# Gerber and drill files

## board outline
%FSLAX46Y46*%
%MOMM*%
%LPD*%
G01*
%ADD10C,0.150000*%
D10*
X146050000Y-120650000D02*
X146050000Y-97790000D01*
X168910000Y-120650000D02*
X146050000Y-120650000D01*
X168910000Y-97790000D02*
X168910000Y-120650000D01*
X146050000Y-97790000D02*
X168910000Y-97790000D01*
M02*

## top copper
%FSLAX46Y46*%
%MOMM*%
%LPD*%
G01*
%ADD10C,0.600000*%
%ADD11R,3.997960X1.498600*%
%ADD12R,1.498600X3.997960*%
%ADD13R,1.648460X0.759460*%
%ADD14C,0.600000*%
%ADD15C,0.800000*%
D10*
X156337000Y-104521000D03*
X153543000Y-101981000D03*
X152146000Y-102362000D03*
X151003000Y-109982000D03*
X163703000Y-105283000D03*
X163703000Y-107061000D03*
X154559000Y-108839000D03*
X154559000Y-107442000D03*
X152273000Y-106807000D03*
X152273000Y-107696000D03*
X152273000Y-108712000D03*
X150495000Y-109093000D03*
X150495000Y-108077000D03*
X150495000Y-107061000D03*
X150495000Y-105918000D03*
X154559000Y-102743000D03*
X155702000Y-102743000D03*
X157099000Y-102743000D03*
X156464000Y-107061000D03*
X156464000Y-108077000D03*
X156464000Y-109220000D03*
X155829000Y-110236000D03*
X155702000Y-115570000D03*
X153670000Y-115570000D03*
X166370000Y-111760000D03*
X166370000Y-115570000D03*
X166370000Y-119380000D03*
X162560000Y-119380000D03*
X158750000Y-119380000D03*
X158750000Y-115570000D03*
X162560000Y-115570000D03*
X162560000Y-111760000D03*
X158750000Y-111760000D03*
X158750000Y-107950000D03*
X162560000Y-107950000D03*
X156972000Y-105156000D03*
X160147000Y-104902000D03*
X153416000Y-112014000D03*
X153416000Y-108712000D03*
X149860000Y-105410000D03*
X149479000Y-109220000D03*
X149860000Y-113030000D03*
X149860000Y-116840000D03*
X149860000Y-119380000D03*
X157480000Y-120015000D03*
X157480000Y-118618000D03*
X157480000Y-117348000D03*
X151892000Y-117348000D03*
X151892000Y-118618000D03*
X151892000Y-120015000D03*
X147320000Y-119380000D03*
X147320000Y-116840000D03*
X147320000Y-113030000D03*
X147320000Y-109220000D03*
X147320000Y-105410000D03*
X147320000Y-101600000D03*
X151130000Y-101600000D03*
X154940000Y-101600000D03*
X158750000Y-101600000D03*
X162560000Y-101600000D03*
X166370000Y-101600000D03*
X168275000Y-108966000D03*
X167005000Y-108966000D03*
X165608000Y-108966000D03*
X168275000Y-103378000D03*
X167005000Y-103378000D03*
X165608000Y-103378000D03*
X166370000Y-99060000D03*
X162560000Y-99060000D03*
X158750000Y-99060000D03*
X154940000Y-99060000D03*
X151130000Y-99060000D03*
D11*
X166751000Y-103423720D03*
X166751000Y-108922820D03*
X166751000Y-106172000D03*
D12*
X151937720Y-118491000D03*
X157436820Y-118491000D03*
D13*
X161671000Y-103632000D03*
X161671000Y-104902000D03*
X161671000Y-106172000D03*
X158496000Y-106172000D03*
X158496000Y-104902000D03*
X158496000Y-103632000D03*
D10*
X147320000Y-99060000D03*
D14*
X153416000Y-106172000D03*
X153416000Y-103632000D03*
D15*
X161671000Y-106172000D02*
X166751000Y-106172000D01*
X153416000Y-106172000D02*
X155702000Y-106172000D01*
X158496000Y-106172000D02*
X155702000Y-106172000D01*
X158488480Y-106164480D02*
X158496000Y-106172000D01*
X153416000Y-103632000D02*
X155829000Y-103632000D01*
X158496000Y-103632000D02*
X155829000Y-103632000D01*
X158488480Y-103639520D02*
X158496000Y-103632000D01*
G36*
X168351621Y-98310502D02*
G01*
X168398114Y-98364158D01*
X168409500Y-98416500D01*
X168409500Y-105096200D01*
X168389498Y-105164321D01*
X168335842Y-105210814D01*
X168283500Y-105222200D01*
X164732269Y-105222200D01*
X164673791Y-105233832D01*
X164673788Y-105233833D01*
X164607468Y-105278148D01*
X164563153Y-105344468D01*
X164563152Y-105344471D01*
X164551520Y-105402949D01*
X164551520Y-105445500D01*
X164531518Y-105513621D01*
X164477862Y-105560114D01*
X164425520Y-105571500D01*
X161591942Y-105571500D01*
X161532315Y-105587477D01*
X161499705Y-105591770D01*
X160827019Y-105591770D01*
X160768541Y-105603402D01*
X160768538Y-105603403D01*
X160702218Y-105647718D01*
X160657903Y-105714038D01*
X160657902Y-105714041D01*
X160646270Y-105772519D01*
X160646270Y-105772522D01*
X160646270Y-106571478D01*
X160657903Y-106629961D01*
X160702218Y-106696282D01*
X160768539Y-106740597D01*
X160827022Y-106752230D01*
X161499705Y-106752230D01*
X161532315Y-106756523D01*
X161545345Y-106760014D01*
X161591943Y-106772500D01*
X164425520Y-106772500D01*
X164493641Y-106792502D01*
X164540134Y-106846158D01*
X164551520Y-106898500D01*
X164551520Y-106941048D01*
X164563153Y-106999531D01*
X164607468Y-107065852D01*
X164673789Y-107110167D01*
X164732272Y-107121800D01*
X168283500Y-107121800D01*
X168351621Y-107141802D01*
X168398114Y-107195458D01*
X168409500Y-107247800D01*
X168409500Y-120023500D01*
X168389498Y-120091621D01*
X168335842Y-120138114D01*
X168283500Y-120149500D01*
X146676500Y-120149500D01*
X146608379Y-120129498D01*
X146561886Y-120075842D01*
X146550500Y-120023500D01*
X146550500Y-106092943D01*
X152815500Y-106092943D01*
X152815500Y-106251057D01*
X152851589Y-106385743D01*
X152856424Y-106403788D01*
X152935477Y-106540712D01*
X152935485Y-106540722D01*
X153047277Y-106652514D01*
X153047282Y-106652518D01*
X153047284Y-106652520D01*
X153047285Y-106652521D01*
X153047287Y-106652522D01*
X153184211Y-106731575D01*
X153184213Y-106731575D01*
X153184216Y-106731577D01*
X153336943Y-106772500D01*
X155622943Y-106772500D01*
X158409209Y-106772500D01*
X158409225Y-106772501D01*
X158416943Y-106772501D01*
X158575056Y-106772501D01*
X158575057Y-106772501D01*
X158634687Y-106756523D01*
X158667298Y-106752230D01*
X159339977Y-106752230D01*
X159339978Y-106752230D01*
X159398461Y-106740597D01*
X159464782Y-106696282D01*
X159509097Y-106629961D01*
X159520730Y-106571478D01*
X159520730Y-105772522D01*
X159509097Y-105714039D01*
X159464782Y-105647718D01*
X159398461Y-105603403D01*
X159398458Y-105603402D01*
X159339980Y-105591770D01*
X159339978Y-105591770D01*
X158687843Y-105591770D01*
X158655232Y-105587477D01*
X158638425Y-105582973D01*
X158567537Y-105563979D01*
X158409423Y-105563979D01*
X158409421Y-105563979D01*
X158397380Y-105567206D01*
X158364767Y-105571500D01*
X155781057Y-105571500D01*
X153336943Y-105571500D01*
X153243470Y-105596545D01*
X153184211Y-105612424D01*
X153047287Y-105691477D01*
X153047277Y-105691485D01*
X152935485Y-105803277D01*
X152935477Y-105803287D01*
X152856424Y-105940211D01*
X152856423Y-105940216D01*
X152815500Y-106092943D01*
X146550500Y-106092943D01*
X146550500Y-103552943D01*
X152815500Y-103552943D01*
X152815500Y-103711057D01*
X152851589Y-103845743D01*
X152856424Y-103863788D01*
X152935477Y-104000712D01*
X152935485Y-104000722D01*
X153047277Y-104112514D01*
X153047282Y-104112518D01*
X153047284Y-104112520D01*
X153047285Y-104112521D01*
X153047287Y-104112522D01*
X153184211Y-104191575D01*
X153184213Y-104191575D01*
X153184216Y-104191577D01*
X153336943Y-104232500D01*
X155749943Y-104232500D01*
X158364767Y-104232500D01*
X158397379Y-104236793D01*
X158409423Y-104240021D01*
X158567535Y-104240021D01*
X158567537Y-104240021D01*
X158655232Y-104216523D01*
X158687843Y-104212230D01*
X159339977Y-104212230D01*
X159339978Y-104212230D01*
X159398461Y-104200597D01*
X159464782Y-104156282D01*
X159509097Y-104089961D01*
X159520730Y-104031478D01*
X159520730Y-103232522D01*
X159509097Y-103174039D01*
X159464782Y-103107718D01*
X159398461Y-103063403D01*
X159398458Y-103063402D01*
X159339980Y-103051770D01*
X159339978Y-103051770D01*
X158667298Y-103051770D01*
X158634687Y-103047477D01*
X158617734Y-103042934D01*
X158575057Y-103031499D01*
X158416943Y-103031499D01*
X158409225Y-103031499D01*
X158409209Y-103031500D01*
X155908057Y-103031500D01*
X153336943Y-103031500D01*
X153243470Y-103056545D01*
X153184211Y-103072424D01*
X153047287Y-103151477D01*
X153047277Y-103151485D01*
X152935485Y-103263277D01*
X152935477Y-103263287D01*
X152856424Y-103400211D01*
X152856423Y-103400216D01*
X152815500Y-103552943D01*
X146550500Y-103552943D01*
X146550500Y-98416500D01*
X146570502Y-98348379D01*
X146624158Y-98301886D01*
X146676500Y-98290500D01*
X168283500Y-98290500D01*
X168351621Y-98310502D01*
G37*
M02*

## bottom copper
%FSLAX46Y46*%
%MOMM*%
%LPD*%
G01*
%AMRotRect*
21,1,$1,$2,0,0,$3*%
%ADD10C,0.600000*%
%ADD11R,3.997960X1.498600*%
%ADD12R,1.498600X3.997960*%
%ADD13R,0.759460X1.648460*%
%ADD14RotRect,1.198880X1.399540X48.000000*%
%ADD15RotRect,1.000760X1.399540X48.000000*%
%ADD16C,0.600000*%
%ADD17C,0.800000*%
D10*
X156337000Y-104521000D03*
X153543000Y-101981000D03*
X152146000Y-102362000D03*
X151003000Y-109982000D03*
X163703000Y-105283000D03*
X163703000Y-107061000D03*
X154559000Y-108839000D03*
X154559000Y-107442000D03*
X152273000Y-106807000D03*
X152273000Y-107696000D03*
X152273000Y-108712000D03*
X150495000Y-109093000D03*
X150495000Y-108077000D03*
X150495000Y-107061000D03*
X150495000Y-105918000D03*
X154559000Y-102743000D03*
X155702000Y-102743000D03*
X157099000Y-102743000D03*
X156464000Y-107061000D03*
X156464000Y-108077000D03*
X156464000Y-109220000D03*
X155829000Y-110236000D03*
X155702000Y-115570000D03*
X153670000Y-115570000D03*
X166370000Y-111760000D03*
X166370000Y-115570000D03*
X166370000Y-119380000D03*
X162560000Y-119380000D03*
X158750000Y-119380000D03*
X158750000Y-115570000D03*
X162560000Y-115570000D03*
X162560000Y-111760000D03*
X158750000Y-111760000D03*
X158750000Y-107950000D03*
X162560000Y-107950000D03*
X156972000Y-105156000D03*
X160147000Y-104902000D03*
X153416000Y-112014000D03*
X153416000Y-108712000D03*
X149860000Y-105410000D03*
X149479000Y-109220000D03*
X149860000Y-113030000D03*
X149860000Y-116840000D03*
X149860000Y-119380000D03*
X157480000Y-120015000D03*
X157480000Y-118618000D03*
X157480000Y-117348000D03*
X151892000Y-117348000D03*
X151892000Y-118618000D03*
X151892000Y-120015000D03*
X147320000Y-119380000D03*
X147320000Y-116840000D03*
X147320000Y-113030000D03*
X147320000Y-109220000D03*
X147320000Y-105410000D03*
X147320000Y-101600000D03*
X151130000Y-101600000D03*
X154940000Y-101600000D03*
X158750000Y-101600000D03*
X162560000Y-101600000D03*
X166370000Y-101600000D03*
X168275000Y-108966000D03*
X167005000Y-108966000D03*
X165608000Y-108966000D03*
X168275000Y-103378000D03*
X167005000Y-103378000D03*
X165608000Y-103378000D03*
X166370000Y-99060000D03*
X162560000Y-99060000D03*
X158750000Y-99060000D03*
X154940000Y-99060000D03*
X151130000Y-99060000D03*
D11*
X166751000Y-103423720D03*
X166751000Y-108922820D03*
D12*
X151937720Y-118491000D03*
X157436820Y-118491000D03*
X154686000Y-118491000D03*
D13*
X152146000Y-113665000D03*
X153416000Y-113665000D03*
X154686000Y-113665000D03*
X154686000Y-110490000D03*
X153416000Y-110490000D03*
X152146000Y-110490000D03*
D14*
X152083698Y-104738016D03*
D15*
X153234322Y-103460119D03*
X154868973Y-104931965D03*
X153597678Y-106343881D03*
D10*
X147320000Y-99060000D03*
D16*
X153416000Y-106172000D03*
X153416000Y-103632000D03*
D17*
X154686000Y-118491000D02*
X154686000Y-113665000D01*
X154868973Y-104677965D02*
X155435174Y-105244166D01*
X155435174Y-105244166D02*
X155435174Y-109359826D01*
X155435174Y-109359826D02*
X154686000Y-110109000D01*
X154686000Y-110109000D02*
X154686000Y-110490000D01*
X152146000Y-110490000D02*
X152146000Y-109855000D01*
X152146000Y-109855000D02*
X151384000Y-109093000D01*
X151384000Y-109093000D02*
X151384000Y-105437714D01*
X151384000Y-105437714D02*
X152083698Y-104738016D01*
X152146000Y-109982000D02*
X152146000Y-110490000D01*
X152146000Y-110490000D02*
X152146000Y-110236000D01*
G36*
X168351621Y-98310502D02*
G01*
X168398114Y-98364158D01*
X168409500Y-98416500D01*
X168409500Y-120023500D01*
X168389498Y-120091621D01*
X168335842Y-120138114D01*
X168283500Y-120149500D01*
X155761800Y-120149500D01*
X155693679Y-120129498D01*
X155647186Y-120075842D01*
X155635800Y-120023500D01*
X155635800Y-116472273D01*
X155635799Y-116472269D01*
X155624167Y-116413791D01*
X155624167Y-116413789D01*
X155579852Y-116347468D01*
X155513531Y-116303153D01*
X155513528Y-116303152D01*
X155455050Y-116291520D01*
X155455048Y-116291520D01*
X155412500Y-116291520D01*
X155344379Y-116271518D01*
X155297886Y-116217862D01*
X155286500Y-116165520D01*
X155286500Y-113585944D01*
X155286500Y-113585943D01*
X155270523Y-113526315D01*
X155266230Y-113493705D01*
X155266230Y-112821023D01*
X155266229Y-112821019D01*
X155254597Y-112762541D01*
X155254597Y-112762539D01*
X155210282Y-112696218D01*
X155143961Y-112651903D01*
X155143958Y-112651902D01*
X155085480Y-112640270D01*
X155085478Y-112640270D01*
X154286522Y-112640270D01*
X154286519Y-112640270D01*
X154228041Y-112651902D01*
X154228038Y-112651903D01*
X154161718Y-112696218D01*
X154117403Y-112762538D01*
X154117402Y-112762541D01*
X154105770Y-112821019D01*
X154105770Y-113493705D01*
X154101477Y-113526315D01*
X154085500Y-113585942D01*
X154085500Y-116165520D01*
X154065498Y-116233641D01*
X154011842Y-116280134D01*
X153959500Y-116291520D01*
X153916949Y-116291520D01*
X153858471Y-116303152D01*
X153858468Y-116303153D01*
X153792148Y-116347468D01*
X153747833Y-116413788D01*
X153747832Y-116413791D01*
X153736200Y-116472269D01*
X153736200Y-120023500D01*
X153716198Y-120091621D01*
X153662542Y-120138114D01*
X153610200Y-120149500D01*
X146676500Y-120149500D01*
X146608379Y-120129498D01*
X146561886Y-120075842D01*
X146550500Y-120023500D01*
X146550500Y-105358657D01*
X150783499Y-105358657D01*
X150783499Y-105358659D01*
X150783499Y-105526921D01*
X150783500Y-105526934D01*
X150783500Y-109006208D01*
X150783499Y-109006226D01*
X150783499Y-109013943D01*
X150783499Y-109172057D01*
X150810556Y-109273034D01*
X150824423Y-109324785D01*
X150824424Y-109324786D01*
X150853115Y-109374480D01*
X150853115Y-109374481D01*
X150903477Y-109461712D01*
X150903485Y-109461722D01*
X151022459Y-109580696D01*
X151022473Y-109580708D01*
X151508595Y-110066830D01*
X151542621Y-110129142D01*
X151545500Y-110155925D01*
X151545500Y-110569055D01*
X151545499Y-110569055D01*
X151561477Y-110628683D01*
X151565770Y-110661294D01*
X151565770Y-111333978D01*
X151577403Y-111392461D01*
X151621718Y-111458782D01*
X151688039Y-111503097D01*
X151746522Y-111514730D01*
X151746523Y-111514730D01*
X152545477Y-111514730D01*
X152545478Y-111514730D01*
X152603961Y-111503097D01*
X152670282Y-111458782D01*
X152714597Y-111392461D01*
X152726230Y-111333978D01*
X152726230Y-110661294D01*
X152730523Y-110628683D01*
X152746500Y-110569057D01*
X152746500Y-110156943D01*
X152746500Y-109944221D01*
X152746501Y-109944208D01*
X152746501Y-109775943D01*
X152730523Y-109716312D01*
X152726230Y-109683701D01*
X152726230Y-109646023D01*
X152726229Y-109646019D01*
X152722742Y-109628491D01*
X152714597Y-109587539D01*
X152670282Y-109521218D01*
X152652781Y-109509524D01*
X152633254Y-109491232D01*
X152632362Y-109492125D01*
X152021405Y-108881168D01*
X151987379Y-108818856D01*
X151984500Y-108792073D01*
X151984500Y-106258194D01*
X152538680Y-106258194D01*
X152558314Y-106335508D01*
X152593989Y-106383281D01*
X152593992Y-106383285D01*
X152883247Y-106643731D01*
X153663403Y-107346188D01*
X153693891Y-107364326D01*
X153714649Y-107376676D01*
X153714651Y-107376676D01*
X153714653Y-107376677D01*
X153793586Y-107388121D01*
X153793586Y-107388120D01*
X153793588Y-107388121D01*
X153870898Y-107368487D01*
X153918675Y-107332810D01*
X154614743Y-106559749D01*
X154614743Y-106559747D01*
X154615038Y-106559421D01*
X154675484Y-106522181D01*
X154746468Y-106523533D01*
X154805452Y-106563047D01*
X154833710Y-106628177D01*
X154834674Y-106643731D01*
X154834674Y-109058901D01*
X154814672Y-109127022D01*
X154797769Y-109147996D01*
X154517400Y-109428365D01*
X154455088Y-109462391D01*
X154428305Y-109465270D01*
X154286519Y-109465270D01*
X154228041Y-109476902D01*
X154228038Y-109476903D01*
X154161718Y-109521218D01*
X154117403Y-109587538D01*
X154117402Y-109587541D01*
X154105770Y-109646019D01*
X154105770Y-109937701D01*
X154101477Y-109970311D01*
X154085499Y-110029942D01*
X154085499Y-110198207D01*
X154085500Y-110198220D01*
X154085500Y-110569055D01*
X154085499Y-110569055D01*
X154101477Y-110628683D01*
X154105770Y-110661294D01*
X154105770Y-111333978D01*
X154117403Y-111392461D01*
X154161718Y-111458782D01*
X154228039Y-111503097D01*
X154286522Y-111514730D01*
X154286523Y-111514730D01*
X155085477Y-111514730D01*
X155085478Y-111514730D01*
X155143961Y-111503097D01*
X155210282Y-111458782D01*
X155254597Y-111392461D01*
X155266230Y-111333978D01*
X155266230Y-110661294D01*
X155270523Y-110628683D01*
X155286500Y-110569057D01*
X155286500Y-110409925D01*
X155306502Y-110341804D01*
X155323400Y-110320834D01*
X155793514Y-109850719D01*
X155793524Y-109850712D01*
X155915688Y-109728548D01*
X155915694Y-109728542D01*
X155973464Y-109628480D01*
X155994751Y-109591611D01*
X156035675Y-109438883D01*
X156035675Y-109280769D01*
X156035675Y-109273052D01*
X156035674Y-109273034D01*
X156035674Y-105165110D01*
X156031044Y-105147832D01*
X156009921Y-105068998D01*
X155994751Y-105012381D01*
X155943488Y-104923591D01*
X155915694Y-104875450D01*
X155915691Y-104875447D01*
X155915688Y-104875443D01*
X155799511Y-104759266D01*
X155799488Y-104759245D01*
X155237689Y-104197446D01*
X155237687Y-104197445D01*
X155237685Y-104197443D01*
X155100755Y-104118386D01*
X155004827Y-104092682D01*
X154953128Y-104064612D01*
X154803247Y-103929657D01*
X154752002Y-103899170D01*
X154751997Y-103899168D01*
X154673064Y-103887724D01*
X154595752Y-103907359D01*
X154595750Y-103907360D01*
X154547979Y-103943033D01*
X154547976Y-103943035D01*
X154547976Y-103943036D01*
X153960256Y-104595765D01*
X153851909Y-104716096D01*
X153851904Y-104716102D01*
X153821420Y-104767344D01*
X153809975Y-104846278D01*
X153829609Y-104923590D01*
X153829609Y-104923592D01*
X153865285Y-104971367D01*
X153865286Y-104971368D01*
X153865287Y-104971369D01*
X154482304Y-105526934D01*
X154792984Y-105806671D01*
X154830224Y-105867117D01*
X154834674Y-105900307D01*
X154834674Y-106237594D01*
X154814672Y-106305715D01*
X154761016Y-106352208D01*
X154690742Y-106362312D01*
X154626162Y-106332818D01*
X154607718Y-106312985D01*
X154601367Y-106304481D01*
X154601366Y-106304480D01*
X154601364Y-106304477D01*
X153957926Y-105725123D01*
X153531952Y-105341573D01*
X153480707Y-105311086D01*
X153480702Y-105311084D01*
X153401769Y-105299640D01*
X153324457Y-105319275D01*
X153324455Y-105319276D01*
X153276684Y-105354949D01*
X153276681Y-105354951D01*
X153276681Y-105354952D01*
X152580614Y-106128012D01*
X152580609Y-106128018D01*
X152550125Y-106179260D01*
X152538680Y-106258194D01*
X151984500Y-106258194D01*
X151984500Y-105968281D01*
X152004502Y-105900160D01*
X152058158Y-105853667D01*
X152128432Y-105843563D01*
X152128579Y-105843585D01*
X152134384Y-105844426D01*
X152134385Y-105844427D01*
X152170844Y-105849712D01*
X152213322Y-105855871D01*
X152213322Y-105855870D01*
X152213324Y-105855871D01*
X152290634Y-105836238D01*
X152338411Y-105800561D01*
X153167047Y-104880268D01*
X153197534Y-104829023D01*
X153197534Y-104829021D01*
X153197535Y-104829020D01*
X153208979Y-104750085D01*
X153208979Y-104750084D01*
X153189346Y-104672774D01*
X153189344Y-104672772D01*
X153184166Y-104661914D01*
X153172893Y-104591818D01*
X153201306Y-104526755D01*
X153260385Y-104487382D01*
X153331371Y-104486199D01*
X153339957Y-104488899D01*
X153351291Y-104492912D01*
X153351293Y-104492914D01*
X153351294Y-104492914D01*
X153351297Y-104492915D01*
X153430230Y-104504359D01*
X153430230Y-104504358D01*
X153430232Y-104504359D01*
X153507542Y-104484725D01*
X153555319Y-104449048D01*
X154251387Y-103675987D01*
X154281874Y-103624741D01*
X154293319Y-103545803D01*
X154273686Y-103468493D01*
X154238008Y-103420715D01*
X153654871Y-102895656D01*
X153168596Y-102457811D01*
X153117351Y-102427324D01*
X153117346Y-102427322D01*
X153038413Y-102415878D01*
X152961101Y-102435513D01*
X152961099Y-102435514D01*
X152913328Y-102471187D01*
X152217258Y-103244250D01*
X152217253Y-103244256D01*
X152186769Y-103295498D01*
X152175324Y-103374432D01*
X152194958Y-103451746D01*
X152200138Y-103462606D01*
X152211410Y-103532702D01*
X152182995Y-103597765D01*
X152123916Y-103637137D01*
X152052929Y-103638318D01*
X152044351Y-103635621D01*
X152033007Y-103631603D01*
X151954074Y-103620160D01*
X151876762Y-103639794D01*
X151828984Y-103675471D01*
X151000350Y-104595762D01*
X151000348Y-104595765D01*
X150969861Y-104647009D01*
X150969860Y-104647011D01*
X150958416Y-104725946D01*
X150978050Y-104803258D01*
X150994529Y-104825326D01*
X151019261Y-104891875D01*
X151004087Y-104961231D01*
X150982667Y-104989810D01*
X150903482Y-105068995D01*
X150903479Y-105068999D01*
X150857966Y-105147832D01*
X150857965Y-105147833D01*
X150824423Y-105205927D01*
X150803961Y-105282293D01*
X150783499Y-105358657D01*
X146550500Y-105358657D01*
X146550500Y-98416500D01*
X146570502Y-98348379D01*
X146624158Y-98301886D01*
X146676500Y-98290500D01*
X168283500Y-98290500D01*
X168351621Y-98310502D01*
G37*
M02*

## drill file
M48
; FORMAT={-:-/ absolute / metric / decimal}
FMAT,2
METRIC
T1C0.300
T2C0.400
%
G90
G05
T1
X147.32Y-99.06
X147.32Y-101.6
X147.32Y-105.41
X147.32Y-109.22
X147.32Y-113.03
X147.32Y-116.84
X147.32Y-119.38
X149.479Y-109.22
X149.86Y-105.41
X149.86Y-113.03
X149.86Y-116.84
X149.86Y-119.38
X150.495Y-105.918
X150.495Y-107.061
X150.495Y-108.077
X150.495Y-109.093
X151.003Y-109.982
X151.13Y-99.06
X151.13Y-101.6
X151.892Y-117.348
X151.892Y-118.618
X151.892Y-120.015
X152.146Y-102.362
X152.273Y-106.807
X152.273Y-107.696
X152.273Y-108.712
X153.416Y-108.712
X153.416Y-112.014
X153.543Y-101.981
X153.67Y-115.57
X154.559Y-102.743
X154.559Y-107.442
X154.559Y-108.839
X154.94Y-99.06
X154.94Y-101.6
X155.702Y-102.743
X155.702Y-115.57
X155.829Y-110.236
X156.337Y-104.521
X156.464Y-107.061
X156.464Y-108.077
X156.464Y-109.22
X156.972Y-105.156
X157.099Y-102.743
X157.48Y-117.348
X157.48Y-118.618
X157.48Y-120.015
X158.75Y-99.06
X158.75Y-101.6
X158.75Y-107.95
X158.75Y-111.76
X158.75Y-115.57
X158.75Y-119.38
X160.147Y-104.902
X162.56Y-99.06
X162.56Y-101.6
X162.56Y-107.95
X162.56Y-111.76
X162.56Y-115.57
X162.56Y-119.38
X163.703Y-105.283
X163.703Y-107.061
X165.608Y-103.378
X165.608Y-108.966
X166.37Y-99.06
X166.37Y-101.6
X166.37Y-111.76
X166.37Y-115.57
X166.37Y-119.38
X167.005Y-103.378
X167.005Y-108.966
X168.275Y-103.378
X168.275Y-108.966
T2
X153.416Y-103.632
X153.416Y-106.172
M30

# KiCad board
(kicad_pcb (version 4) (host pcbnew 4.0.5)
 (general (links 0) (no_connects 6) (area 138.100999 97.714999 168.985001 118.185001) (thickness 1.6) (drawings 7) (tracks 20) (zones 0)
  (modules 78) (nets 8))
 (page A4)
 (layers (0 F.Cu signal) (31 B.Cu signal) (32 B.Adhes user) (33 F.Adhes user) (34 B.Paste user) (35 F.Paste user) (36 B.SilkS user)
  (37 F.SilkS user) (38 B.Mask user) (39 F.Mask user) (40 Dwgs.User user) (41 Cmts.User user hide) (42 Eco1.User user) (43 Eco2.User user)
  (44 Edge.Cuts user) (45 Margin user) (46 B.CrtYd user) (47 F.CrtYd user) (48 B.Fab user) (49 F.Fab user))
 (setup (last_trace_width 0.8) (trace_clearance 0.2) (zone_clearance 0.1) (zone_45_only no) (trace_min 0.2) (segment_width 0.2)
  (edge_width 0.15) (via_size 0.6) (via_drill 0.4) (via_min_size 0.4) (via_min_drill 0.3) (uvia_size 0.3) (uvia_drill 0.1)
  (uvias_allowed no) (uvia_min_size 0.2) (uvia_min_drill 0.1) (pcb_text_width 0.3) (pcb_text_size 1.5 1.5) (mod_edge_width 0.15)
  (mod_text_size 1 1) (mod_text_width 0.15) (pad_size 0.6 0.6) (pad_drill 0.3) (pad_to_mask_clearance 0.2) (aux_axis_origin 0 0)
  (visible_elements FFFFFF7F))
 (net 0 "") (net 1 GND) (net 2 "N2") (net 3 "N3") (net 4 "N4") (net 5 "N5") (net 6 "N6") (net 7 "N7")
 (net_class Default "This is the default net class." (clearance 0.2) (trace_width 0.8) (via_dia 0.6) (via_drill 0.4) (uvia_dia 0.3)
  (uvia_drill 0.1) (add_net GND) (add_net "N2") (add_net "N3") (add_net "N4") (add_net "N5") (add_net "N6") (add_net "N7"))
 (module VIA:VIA (layer F.Cu) (at 156.337 104.521)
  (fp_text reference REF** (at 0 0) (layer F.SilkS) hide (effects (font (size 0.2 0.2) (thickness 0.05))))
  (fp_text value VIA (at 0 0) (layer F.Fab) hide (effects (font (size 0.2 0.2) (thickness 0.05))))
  (pad 1 thru_hole circle (at 0 0) (size 0.6 0.6) (drill 0.3) (layers *.Cu) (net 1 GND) (zone_connect 2)))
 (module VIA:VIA (layer F.Cu) (at 153.543 101.981)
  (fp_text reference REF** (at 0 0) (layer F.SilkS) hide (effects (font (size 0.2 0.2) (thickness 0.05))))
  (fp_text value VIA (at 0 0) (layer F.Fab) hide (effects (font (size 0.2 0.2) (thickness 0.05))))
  (pad 1 thru_hole circle (at 0 0) (size 0.6 0.6) (drill 0.3) (layers *.Cu) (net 1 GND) (zone_connect 2)))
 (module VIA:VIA (layer F.Cu) (at 152.146 102.362)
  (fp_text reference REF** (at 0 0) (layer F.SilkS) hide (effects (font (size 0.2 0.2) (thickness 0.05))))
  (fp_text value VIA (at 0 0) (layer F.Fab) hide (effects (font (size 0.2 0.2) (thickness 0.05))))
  (pad 1 thru_hole circle (at 0 0) (size 0.6 0.6) (drill 0.3) (layers *.Cu) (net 1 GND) (zone_connect 2)))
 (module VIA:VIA (layer F.Cu) (at 151.003 109.982)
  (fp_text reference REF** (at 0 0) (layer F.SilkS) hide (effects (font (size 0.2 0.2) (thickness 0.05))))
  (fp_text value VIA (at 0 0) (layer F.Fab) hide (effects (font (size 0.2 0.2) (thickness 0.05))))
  (pad 1 thru_hole circle (at 0 0) (size 0.6 0.6) (drill 0.3) (layers *.Cu) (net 1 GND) (zone_connect 2)))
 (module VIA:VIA (layer F.Cu) (at 163.703 105.283)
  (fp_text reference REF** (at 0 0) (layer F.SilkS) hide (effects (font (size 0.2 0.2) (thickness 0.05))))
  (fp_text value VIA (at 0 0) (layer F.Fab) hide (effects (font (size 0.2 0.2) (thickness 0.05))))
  (pad 1 thru_hole circle (at 0 0) (size 0.6 0.6) (drill 0.3) (layers *.Cu) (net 1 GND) (zone_connect 2)))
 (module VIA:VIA (layer F.Cu) (at 163.703 107.061)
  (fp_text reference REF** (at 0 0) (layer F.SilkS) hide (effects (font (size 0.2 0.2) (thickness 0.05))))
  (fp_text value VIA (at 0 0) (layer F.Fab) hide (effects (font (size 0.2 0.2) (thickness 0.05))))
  (pad 1 thru_hole circle (at 0 0) (size 0.6 0.6) (drill 0.3) (layers *.Cu) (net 1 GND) (zone_connect 2)))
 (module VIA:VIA (layer F.Cu) (at 154.559 108.839)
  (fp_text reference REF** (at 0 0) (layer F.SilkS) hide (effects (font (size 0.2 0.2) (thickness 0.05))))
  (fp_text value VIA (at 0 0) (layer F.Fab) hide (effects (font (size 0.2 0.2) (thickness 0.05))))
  (pad 1 thru_hole circle (at 0 0) (size 0.6 0.6) (drill 0.3) (layers *.Cu) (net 1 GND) (zone_connect 2)))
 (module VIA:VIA (layer F.Cu) (at 154.559 107.442)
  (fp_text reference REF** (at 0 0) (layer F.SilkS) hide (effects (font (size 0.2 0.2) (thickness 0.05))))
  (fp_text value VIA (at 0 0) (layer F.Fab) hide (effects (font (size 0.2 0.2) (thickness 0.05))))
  (pad 1 thru_hole circle (at 0 0) (size 0.6 0.6) (drill 0.3) (layers *.Cu) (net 1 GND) (zone_connect 2)))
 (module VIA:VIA (layer F.Cu) (at 152.273 106.807)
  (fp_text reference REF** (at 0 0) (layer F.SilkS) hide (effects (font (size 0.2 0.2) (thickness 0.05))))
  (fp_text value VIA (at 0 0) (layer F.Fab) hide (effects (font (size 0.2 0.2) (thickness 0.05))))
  (pad 1 thru_hole circle (at 0 0) (size 0.6 0.6) (drill 0.3) (layers *.Cu) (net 1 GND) (zone_connect 2)))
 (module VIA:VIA (layer F.Cu) (at 152.273 107.696)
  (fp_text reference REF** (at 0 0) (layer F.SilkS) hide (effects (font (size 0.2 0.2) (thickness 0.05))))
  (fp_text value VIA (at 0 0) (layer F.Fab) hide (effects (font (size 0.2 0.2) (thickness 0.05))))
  (pad 1 thru_hole circle (at 0 0) (size 0.6 0.6) (drill 0.3) (layers *.Cu) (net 1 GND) (zone_connect 2)))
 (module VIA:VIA (layer F.Cu) (at 152.273 108.712)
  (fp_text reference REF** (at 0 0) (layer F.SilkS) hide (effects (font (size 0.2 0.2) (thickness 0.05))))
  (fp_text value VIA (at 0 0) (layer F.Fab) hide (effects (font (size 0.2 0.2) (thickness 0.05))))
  (pad 1 thru_hole circle (at 0 0) (size 0.6 0.6) (drill 0.3) (layers *.Cu) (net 1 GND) (zone_connect 2)))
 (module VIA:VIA (layer F.Cu) (at 150.495 109.093)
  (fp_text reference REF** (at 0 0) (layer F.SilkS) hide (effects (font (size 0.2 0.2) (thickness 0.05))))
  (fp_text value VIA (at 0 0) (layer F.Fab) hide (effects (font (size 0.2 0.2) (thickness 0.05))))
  (pad 1 thru_hole circle (at 0 0) (size 0.6 0.6) (drill 0.3) (layers *.Cu) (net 1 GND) (zone_connect 2)))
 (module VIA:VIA (layer F.Cu) (at 150.495 108.077)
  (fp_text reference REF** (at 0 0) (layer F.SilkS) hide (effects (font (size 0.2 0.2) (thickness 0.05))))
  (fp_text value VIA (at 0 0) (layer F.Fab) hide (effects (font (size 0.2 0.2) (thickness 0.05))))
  (pad 1 thru_hole circle (at 0 0) (size 0.6 0.6) (drill 0.3) (layers *.Cu) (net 1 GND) (zone_connect 2)))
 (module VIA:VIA (layer F.Cu) (at 150.495 107.061)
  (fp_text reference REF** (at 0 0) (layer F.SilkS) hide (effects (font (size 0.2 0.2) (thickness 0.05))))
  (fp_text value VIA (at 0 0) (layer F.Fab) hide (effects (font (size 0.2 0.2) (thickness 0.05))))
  (pad 1 thru_hole circle (at 0 0) (size 0.6 0.6) (drill 0.3) (layers *.Cu) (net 1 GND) (zone_connect 2)))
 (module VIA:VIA (layer F.Cu) (at 150.495 105.918)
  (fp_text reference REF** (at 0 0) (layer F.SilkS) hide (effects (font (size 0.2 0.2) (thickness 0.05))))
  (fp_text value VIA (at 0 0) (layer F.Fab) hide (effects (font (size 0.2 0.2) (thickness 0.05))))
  (pad 1 thru_hole circle (at 0 0) (size 0.6 0.6) (drill 0.3) (layers *.Cu) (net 1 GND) (zone_connect 2)))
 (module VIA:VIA (layer F.Cu) (at 154.559 102.743)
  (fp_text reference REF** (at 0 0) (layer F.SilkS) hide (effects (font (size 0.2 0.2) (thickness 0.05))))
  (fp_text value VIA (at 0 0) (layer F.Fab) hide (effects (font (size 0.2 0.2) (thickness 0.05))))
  (pad 1 thru_hole circle (at 0 0) (size 0.6 0.6) (drill 0.3) (layers *.Cu) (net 1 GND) (zone_connect 2)))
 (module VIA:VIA (layer F.Cu) (at 155.702 102.743)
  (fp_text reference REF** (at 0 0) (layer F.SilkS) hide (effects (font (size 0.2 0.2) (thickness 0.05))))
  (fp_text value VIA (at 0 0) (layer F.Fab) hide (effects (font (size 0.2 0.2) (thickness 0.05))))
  (pad 1 thru_hole circle (at 0 0) (size 0.6 0.6) (drill 0.3) (layers *.Cu) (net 1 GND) (zone_connect 2)))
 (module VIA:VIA (layer F.Cu) (at 157.099 102.743)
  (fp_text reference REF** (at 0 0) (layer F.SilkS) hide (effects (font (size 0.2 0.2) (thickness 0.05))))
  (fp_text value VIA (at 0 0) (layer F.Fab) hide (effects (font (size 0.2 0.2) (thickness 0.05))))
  (pad 1 thru_hole circle (at 0 0) (size 0.6 0.6) (drill 0.3) (layers *.Cu) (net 1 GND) (zone_connect 2)))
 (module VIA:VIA (layer F.Cu) (at 156.464 107.061)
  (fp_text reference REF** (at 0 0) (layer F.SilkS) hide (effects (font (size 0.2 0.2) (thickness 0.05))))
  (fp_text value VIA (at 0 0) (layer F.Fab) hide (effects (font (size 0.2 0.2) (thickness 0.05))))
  (pad 1 thru_hole circle (at 0 0) (size 0.6 0.6) (drill 0.3) (layers *.Cu) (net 1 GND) (zone_connect 2)))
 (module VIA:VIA (layer F.Cu) (at 156.464 108.077)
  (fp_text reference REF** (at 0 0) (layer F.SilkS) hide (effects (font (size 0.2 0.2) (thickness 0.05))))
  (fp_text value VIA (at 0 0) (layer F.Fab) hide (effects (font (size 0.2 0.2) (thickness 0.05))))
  (pad 1 thru_hole circle (at 0 0) (size 0.6 0.6) (drill 0.3) (layers *.Cu) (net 1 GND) (zone_connect 2)))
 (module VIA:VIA (layer F.Cu) (at 156.464 109.22)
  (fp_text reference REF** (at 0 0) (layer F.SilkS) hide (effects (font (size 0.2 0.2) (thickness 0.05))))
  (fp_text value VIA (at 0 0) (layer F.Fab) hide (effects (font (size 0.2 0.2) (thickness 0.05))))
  (pad 1 thru_hole circle (at 0 0) (size 0.6 0.6) (drill 0.3) (layers *.Cu) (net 1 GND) (zone_connect 2)))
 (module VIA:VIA (layer F.Cu) (at 155.829 110.236)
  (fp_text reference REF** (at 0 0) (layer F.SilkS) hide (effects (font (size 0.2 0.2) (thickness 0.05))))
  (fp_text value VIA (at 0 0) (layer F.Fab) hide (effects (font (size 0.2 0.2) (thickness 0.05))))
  (pad 1 thru_hole circle (at 0 0) (size 0.6 0.6) (drill 0.3) (layers *.Cu) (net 1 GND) (zone_connect 2)))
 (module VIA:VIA (layer F.Cu) (at 155.702 115.57)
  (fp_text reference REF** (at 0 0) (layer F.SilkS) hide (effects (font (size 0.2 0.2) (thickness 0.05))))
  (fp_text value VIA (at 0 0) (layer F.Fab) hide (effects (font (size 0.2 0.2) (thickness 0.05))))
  (pad 1 thru_hole circle (at 0 0) (size 0.6 0.6) (drill 0.3) (layers *.Cu) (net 1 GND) (zone_connect 2)))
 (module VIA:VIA (layer F.Cu) (at 153.67 115.57)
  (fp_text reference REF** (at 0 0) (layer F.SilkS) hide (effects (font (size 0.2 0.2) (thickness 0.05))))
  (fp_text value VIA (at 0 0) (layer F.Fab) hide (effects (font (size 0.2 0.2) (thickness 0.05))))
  (pad 1 thru_hole circle (at 0 0) (size 0.6 0.6) (drill 0.3) (layers *.Cu) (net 1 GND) (zone_connect 2)))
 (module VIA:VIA (layer F.Cu) (at 166.37 111.76)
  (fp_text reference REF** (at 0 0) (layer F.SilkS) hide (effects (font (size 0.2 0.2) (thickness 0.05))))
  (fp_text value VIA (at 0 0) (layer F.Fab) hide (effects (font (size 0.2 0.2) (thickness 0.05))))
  (pad 1 thru_hole circle (at 0 0) (size 0.6 0.6) (drill 0.3) (layers *.Cu) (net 1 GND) (zone_connect 2)))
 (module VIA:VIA (layer F.Cu) (at 166.37 115.57)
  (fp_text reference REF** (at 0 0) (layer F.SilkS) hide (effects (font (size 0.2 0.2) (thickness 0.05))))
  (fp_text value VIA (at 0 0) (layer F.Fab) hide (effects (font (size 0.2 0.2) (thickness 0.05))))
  (pad 1 thru_hole circle (at 0 0) (size 0.6 0.6) (drill 0.3) (layers *.Cu) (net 1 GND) (zone_connect 2)))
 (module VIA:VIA (layer F.Cu) (at 166.37 119.38)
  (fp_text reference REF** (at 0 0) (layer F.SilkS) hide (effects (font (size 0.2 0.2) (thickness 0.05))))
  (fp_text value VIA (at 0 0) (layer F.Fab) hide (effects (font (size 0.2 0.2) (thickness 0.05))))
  (pad 1 thru_hole circle (at 0 0) (size 0.6 0.6) (drill 0.3) (layers *.Cu) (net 1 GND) (zone_connect 2)))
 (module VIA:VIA (layer F.Cu) (at 162.56 119.38)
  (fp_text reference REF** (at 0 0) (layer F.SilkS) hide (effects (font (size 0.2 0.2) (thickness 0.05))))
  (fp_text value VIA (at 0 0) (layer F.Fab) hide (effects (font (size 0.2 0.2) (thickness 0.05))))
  (pad 1 thru_hole circle (at 0 0) (size 0.6 0.6) (drill 0.3) (layers *.Cu) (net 1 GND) (zone_connect 2)))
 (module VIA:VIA (layer F.Cu) (at 158.75 119.38)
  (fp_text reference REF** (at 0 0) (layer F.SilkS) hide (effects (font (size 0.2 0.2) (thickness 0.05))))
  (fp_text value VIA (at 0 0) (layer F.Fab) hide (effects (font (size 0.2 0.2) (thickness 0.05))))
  (pad 1 thru_hole circle (at 0 0) (size 0.6 0.6) (drill 0.3) (layers *.Cu) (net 1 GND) (zone_connect 2)))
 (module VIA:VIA (layer F.Cu) (at 158.75 115.57)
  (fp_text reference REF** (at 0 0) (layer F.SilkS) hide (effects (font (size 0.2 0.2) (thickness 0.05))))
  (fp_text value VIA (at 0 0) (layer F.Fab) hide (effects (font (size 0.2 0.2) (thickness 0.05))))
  (pad 1 thru_hole circle (at 0 0) (size 0.6 0.6) (drill 0.3) (layers *.Cu) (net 1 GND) (zone_connect 2)))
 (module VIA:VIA (layer F.Cu) (at 162.56 115.57)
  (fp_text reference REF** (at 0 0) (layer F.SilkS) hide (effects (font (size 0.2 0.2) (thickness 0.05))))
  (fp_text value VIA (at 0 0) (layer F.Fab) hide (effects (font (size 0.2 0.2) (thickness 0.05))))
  (pad 1 thru_hole circle (at 0 0) (size 0.6 0.6) (drill 0.3) (layers *.Cu) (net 1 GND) (zone_connect 2)))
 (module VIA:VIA (layer F.Cu) (at 162.56 111.76)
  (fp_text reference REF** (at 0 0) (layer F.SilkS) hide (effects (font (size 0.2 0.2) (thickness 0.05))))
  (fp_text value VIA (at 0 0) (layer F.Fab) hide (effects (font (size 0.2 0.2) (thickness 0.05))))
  (pad 1 thru_hole circle (at 0 0) (size 0.6 0.6) (drill 0.3) (layers *.Cu) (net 1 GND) (zone_connect 2)))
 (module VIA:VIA (layer F.Cu) (at 158.75 111.76)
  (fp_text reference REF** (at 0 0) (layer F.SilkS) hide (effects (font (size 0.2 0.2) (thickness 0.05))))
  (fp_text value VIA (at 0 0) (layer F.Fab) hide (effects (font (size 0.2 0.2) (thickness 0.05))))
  (pad 1 thru_hole circle (at 0 0) (size 0.6 0.6) (drill 0.3) (layers *.Cu) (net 1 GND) (zone_connect 2)))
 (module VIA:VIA (layer F.Cu) (at 158.75 107.95)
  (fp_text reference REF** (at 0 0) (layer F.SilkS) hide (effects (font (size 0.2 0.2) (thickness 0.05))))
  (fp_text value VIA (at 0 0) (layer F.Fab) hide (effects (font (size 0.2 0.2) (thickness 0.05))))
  (pad 1 thru_hole circle (at 0 0) (size 0.6 0.6) (drill 0.3) (layers *.Cu) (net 1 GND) (zone_connect 2)))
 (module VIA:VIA (layer F.Cu) (at 162.56 107.95)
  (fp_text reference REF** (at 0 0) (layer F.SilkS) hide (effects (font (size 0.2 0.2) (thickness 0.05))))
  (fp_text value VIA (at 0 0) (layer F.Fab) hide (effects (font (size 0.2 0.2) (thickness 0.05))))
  (pad 1 thru_hole circle (at 0 0) (size 0.6 0.6) (drill 0.3) (layers *.Cu) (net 1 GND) (zone_connect 2)))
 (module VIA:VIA (layer F.Cu) (at 156.972 105.156)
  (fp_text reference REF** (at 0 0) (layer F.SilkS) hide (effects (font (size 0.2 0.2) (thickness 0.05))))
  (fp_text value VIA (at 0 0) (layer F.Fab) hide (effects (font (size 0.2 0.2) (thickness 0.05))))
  (pad 1 thru_hole circle (at 0 0) (size 0.6 0.6) (drill 0.3) (layers *.Cu) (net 1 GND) (zone_connect 2)))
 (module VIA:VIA (layer F.Cu) (at 160.147 104.902)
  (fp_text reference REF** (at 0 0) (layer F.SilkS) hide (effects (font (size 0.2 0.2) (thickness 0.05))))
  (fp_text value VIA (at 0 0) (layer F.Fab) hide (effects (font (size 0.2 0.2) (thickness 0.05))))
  (pad 1 thru_hole circle (at 0 0) (size 0.6 0.6) (drill 0.3) (layers *.Cu) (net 1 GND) (zone_connect 2)))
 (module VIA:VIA (layer F.Cu) (at 153.416 112.014)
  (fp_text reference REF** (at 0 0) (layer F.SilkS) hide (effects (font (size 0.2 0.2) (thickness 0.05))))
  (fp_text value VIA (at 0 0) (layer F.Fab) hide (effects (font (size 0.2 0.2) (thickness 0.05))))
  (pad 1 thru_hole circle (at 0 0) (size 0.6 0.6) (drill 0.3) (layers *.Cu) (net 1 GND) (zone_connect 2)))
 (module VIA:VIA (layer F.Cu) (at 153.416 108.712)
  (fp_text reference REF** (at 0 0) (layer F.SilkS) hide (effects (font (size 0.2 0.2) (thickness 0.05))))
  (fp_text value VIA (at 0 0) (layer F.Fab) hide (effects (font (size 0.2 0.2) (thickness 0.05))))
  (pad 1 thru_hole circle (at 0 0) (size 0.6 0.6) (drill 0.3) (layers *.Cu) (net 1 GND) (zone_connect 2)))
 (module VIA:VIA (layer F.Cu) (at 149.86 105.41)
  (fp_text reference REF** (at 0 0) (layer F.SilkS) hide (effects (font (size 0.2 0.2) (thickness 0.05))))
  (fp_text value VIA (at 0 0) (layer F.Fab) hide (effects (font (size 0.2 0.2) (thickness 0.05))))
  (pad 1 thru_hole circle (at 0 0) (size 0.6 0.6) (drill 0.3) (layers *.Cu) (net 1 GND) (zone_connect 2)))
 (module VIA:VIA (layer F.Cu) (at 149.479 109.22)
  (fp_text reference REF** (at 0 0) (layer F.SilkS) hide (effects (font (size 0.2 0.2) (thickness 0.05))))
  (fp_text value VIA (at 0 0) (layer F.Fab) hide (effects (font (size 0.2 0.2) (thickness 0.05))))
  (pad 1 thru_hole circle (at 0 0) (size 0.6 0.6) (drill 0.3) (layers *.Cu) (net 1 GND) (zone_connect 2)))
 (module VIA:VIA (layer F.Cu) (at 149.86 113.03)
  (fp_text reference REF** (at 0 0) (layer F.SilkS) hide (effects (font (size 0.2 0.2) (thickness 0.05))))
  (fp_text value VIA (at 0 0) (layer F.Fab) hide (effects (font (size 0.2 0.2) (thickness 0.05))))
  (pad 1 thru_hole circle (at 0 0) (size 0.6 0.6) (drill 0.3) (layers *.Cu) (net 1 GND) (zone_connect 2)))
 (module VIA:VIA (layer F.Cu) (at 149.86 116.84)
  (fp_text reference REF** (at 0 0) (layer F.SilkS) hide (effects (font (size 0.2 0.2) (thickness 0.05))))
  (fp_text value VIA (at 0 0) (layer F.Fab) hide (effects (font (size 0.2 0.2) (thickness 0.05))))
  (pad 1 thru_hole circle (at 0 0) (size 0.6 0.6) (drill 0.3) (layers *.Cu) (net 1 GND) (zone_connect 2)))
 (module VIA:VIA (layer F.Cu) (at 149.86 119.38)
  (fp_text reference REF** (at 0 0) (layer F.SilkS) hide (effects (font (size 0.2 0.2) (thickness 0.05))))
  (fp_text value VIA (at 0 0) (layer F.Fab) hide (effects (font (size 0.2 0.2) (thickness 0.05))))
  (pad 1 thru_hole circle (at 0 0) (size 0.6 0.6) (drill 0.3) (layers *.Cu) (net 1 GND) (zone_connect 2)))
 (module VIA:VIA (layer F.Cu) (at 157.48 120.015)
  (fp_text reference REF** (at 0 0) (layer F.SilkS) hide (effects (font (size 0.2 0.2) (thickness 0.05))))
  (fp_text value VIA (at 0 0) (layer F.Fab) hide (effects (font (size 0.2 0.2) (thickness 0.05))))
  (pad 1 thru_hole circle (at 0 0) (size 0.6 0.6) (drill 0.3) (layers *.Cu) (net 1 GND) (zone_connect 2)))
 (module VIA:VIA (layer F.Cu) (at 157.48 118.618)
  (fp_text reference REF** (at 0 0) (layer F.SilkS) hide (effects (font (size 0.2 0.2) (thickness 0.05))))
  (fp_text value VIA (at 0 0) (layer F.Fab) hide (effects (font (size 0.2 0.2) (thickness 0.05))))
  (pad 1 thru_hole circle (at 0 0) (size 0.6 0.6) (drill 0.3) (layers *.Cu) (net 1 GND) (zone_connect 2)))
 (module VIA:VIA (layer F.Cu) (at 157.48 117.348)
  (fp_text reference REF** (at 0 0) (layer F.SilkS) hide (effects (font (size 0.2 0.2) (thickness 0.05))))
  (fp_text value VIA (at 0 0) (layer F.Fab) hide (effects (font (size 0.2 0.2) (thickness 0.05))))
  (pad 1 thru_hole circle (at 0 0) (size 0.6 0.6) (drill 0.3) (layers *.Cu) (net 1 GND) (zone_connect 2)))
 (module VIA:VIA (layer F.Cu) (at 151.892 117.348)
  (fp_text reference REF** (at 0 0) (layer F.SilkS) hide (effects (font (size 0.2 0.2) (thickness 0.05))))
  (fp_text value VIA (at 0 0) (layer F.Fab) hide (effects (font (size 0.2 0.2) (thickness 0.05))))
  (pad 1 thru_hole circle (at 0 0) (size 0.6 0.6) (drill 0.3) (layers *.Cu) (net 1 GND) (zone_connect 2)))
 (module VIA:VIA (layer F.Cu) (at 151.892 118.618)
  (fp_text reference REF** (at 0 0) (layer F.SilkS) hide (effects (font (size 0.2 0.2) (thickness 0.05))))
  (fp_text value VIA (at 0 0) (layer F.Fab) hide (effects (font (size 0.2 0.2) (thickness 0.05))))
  (pad 1 thru_hole circle (at 0 0) (size 0.6 0.6) (drill 0.3) (layers *.Cu) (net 1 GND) (zone_connect 2)))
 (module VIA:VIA (layer F.Cu) (at 151.892 120.015)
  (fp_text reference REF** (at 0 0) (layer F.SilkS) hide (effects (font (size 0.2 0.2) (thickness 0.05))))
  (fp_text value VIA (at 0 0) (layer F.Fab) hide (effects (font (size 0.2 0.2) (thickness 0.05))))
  (pad 1 thru_hole circle (at 0 0) (size 0.6 0.6) (drill 0.3) (layers *.Cu) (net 1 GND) (zone_connect 2)))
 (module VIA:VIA (layer F.Cu) (at 147.32 119.38)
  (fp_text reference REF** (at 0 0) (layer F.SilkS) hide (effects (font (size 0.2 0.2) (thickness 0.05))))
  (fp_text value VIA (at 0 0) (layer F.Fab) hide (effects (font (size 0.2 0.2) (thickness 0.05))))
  (pad 1 thru_hole circle (at 0 0) (size 0.6 0.6) (drill 0.3) (layers *.Cu) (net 1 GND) (zone_connect 2)))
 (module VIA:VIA (layer F.Cu) (at 147.32 116.84)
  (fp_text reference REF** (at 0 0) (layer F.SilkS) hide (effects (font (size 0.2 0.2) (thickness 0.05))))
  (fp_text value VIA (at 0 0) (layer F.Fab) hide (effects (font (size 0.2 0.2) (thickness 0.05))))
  (pad 1 thru_hole circle (at 0 0) (size 0.6 0.6) (drill 0.3) (layers *.Cu) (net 1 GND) (zone_connect 2)))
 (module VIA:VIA (layer F.Cu) (at 147.32 113.03)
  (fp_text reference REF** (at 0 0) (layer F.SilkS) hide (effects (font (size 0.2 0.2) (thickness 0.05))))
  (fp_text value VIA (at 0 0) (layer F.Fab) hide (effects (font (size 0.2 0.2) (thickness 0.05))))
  (pad 1 thru_hole circle (at 0 0) (size 0.6 0.6) (drill 0.3) (layers *.Cu) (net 1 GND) (zone_connect 2)))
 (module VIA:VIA (layer F.Cu) (at 147.32 109.22)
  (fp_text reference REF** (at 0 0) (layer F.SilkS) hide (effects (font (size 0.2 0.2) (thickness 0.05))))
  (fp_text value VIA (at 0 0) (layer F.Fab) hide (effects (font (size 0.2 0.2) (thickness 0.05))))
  (pad 1 thru_hole circle (at 0 0) (size 0.6 0.6) (drill 0.3) (layers *.Cu) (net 1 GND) (zone_connect 2)))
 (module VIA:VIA (layer F.Cu) (at 147.32 105.41)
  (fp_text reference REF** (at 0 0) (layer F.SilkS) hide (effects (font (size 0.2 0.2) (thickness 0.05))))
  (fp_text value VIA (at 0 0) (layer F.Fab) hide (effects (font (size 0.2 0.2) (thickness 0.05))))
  (pad 1 thru_hole circle (at 0 0) (size 0.6 0.6) (drill 0.3) (layers *.Cu) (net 1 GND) (zone_connect 2)))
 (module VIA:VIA (layer F.Cu) (at 147.32 101.6)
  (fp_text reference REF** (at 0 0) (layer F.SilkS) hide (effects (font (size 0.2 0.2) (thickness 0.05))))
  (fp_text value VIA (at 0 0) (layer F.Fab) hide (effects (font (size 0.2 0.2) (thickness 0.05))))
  (pad 1 thru_hole circle (at 0 0) (size 0.6 0.6) (drill 0.3) (layers *.Cu) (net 1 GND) (zone_connect 2)))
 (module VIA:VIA (layer F.Cu) (at 151.13 101.6)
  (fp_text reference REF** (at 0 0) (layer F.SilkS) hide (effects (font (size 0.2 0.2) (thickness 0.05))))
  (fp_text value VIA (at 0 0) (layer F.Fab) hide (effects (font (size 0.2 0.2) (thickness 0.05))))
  (pad 1 thru_hole circle (at 0 0) (size 0.6 0.6) (drill 0.3) (layers *.Cu) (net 1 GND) (zone_connect 2)))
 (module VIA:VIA (layer F.Cu) (at 154.94 101.6)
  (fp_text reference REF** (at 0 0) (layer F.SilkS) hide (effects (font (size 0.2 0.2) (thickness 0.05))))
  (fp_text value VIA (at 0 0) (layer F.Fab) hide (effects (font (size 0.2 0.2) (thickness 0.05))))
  (pad 1 thru_hole circle (at 0 0) (size 0.6 0.6) (drill 0.3) (layers *.Cu) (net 1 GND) (zone_connect 2)))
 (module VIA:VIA (layer F.Cu) (at 158.75 101.6)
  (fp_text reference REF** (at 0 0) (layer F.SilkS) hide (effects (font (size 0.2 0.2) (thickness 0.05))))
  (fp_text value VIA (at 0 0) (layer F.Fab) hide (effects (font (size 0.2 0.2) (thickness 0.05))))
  (pad 1 thru_hole circle (at 0 0) (size 0.6 0.6) (drill 0.3) (layers *.Cu) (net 1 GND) (zone_connect 2)))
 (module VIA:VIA (layer F.Cu) (at 162.56 101.6)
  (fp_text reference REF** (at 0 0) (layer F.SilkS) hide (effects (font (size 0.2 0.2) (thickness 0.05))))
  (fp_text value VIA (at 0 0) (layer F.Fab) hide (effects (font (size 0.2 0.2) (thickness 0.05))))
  (pad 1 thru_hole circle (at 0 0) (size 0.6 0.6) (drill 0.3) (layers *.Cu) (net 1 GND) (zone_connect 2)))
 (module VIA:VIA (layer F.Cu) (at 166.37 101.6)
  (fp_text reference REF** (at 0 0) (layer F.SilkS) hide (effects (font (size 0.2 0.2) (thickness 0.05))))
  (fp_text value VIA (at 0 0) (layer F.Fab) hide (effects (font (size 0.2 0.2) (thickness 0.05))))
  (pad 1 thru_hole circle (at 0 0) (size 0.6 0.6) (drill 0.3) (layers *.Cu) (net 1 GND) (zone_connect 2)))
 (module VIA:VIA (layer F.Cu) (at 168.275 108.966)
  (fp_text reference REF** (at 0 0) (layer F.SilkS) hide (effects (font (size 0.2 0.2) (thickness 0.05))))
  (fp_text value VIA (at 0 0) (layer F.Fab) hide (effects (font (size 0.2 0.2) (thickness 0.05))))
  (pad 1 thru_hole circle (at 0 0) (size 0.6 0.6) (drill 0.3) (layers *.Cu) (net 1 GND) (zone_connect 2)))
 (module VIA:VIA (layer F.Cu) (at 167.005 108.966)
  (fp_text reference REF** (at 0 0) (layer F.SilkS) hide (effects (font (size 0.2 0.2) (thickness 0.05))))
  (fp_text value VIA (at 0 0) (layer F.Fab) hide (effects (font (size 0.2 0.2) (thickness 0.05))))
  (pad 1 thru_hole circle (at 0 0) (size 0.6 0.6) (drill 0.3) (layers *.Cu) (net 1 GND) (zone_connect 2)))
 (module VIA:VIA (layer F.Cu) (at 165.608 108.966)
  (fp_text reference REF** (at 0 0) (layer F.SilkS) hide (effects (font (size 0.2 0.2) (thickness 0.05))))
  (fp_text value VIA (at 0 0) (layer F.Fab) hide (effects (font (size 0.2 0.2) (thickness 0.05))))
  (pad 1 thru_hole circle (at 0 0) (size 0.6 0.6) (drill 0.3) (layers *.Cu) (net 1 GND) (zone_connect 2)))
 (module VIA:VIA (layer F.Cu) (at 168.275 103.378)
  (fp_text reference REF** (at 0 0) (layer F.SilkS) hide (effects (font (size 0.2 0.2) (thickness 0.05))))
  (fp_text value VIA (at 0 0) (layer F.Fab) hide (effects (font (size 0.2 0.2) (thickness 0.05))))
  (pad 1 thru_hole circle (at 0 0) (size 0.6 0.6) (drill 0.3) (layers *.Cu) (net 1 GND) (zone_connect 2)))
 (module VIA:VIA (layer F.Cu) (at 167.005 103.378)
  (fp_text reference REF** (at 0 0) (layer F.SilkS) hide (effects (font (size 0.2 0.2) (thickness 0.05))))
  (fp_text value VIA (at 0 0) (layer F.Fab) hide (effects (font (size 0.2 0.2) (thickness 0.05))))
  (pad 1 thru_hole circle (at 0 0) (size 0.6 0.6) (drill 0.3) (layers *.Cu) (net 1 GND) (zone_connect 2)))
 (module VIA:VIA (layer F.Cu) (at 165.608 103.378)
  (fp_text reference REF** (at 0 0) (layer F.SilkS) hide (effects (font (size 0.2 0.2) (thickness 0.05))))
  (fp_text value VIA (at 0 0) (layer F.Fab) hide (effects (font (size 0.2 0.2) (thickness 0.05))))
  (pad 1 thru_hole circle (at 0 0) (size 0.6 0.6) (drill 0.3) (layers *.Cu) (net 1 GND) (zone_connect 2)))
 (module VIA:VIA (layer F.Cu) (at 166.37 99.06)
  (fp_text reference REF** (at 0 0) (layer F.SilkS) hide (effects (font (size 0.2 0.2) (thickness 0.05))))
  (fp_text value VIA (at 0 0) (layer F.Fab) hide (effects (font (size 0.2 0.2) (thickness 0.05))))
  (pad 1 thru_hole circle (at 0 0) (size 0.6 0.6) (drill 0.3) (layers *.Cu) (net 1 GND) (zone_connect 2)))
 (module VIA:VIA (layer F.Cu) (at 162.56 99.06)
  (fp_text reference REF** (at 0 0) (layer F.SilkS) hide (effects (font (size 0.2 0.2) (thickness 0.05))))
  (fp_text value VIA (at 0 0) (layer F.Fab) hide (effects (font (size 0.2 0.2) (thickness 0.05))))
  (pad 1 thru_hole circle (at 0 0) (size 0.6 0.6) (drill 0.3) (layers *.Cu) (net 1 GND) (zone_connect 2)))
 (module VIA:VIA (layer F.Cu) (at 158.75 99.06)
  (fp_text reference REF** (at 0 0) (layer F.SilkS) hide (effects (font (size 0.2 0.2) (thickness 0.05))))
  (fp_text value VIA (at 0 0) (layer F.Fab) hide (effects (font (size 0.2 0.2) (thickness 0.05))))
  (pad 1 thru_hole circle (at 0 0) (size 0.6 0.6) (drill 0.3) (layers *.Cu) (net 1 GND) (zone_connect 2)))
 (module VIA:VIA (layer F.Cu) (at 154.94 99.06)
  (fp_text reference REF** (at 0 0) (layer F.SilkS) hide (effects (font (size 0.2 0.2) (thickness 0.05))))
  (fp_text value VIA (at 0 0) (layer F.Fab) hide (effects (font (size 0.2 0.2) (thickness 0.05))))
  (pad 1 thru_hole circle (at 0 0) (size 0.6 0.6) (drill 0.3) (layers *.Cu) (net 1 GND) (zone_connect 2)))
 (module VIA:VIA (layer F.Cu) (at 151.13 99.06)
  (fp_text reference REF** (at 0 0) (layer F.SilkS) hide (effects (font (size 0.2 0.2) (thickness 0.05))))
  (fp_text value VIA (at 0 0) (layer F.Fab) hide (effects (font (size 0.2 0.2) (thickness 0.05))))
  (pad 1 thru_hole circle (at 0 0) (size 0.6 0.6) (drill 0.3) (layers *.Cu) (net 1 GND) (zone_connect 2)))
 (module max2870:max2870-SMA (layer F.Cu) (at 166.751 103.42372 270)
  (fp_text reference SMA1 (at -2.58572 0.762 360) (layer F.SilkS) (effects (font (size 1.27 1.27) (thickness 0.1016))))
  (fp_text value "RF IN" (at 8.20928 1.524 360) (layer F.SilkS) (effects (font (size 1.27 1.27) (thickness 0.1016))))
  (pad GND@ smd rect (at 0 0) (size 3.99796 1.4986) (layers F.Cu F.Paste F.Mask) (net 1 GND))
  (pad GND@ smd rect (at 5.4991 0) (size 3.99796 1.4986) (layers F.Cu F.Paste F.Mask) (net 1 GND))
  (pad GND@ smd rect (at 0 0) (size 3.99796 1.4986) (layers B.Cu B.Mask) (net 1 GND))
  (pad GND@ smd rect (at 5.4991 0) (size 3.99796 1.4986) (layers B.Cu B.Mask) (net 1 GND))
  (pad SIGN smd rect (at 2.74828 0) (size 3.99796 1.4986) (layers F.Cu F.Paste F.Mask) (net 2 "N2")))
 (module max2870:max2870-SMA (layer B.Cu) (at 151.93772 118.491)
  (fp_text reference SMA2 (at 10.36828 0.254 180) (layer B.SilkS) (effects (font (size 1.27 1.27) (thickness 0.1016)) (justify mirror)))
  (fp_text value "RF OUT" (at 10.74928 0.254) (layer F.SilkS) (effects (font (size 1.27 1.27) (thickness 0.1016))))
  (pad GND@ smd rect (at 0 0 270) (size 3.99796 1.4986) (layers B.Cu B.Paste B.Mask) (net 1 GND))
  (pad GND@ smd rect (at 5.4991 0 270) (size 3.99796 1.4986) (layers B.Cu B.Paste B.Mask) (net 1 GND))
  (pad GND@ smd rect (at 0 0 270) (size 3.99796 1.4986) (layers F.Cu F.Mask) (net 1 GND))
  (pad GND@ smd rect (at 5.4991 0 270) (size 3.99796 1.4986) (layers F.Cu F.Mask) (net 1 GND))
  (pad SIGN smd rect (at 2.74828 0 270) (size 3.99796 1.4986) (layers B.Cu B.Paste B.Mask) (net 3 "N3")))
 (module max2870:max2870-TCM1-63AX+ (layer F.Cu) (at 160.401 104.902 270)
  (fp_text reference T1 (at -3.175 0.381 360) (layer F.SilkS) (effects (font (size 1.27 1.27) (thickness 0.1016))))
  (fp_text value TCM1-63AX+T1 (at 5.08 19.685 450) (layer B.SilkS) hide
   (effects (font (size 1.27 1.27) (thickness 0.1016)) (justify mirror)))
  (pad 1 smd rect (at -1.27 -1.27 90) (size 0.75946 1.64846) (layers F.Cu F.Paste F.Mask) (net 1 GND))
  (pad 2 smd rect (at 0 -1.27 90) (size 0.75946 1.64846) (layers F.Cu F.Paste F.Mask) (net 1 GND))
  (pad 3 smd rect (at 1.27 -1.27 90) (size 0.75946 1.64846) (layers F.Cu F.Paste F.Mask) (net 2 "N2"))
  (pad 4 smd rect (at 1.27 1.905 90) (size 0.75946 1.64846) (layers F.Cu F.Paste F.Mask) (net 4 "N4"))
  (pad 5 smd rect (at 0 1.905 90) (size 0.75946 1.64846) (layers F.Cu F.Paste F.Mask) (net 1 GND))
  (pad 6 smd rect (at -1.27 1.905 90) (size 0.75946 1.64846) (layers F.Cu F.Paste F.Mask) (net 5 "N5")))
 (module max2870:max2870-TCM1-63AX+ (layer B.Cu) (at 153.416 112.395)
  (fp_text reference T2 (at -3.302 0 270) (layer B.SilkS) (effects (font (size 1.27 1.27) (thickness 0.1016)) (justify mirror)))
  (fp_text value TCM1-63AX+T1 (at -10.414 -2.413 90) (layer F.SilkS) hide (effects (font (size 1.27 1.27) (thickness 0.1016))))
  (pad 1 smd rect (at -1.27 1.27 180) (size 0.75946 1.64846) (layers B.Cu B.Paste B.Mask) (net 1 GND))
  (pad 2 smd rect (at 0 1.27 180) (size 0.75946 1.64846) (layers B.Cu B.Paste B.Mask) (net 1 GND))
  (pad 3 smd rect (at 1.27 1.27 180) (size 0.75946 1.64846) (layers B.Cu B.Paste B.Mask) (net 3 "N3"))
  (pad 4 smd rect (at 1.27 -1.905 180) (size 0.75946 1.64846) (layers B.Cu B.Paste B.Mask) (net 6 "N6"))
  (pad 5 smd rect (at 0 -1.905 180) (size 0.75946 1.64846) (layers B.Cu B.Paste B.Mask) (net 1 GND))
  (pad 6 smd rect (at -1.27 -1.905 180) (size 0.75946 1.64846) (layers B.Cu B.Paste B.Mask) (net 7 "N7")))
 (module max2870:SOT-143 (layer B.Cu) (at 153.416 104.902 48)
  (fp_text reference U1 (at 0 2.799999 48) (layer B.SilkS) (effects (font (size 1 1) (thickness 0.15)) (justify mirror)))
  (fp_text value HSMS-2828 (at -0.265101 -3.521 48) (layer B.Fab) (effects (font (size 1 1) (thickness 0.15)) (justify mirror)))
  (pad 1 smd rect (at -0.76962 -1.09982 48) (size 1.19888 1.39954) (layers B.Cu B.Paste B.Mask) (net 7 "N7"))
  (pad 2 smd rect (at 0.94996 -1.09982 48) (size 1.00076 1.39954) (layers B.Cu B.Paste B.Mask) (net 5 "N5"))
  (pad 4 smd rect (at 0.94996 1.09982 48) (size 1.00076 1.39954) (layers B.Cu B.Paste B.Mask) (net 6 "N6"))
  (pad 3 smd rect (at -0.94996 1.09982 48) (size 1.00076 1.39954) (layers B.Cu B.Paste B.Mask) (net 4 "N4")))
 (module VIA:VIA (layer F.Cu) (at 147.32 99.06)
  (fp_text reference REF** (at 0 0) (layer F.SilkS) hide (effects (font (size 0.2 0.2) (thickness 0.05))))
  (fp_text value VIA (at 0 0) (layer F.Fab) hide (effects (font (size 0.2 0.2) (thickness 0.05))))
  (pad 1 thru_hole circle (at 0 0) (size 0.6 0.6) (drill 0.3) (layers *.Cu) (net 1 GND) (zone_connect 2)))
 (gr_line (start 146.05 120.65) (end 146.05 97.79) (layer Edge.Cuts) (width 0.15))
 (gr_line (start 168.91 120.65) (end 146.05 120.65) (layer Edge.Cuts) (width 0.15))
 (gr_line (start 168.91 97.79) (end 168.91 120.65) (layer Edge.Cuts) (width 0.15))
 (gr_line (start 146.05 97.79) (end 168.91 97.79) (layer Edge.Cuts) (width 0.15))
 (segment (start 161.671 106.172) (end 166.751 106.172) (width 0.8) (layer F.Cu) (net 2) (status 30))
 (segment (start 154.686 118.491) (end 154.686 113.665) (width 0.8) (layer B.Cu) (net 3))
 (segment (start 153.416 106.172) (end 155.702 106.172) (width 0.8) (layer F.Cu) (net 4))
 (segment (start 158.496 106.172) (end 155.702 106.172) (width 0.8) (layer F.Cu) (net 4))
 (via (at 153.416 106.172) (size 0.6) (drill 0.4) (layers F.Cu B.Cu) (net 4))
 (segment (start 158.48848 106.16448) (end 158.496 106.172) (width 0.8) (layer F.Cu) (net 4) (status 30))
 (segment (start 153.416 103.632) (end 155.829 103.632) (width 0.8) (layer F.Cu) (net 5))
 (segment (start 158.496 103.632) (end 155.829 103.632) (width 0.8) (layer F.Cu) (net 5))
 (via (at 153.416 103.632) (size 0.6) (drill 0.4) (layers F.Cu B.Cu) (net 5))
 (segment (start 158.48848 103.63952) (end 158.496 103.632) (width 0.8) (layer F.Cu) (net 5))
 (segment (start 154.868973 104.677965) (end 155.435174 105.244166) (width 0.8) (layer B.Cu) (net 6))
 (segment (start 155.435174 105.244166) (end 155.435174 109.359826) (width 0.8) (layer B.Cu) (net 6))
 (segment (start 155.435174 109.359826) (end 154.686 110.109) (width 0.8) (layer B.Cu) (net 6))
 (segment (start 154.686 110.109) (end 154.686 110.49) (width 0.8) (layer B.Cu) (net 6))
 (segment (start 152.146 110.49) (end 152.146 109.855) (width 0.8) (layer B.Cu) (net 7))
 (segment (start 152.146 109.855) (end 151.384 109.093) (width 0.8) (layer B.Cu) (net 7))
 (segment (start 151.384 109.093) (end 151.384 105.437714) (width 0.8) (layer B.Cu) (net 7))
 (segment (start 151.384 105.437714) (end 152.083698 104.738016) (width 0.8) (layer B.Cu) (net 7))
 (segment (start 152.146 109.982) (end 152.146 110.49) (width 0.8) (layer B.Cu) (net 7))
 (segment (start 152.146 110.49) (end 152.146 110.236) (width 0.8) (layer B.Cu) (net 7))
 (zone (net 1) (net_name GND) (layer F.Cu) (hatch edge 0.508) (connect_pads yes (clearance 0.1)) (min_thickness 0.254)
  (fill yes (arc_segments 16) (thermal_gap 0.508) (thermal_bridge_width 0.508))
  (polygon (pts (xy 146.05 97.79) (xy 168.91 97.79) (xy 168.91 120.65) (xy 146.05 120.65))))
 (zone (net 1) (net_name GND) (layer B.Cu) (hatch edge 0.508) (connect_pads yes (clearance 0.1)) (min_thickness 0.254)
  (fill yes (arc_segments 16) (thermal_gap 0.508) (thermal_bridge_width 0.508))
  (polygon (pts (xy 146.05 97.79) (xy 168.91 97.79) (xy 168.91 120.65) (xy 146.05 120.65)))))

